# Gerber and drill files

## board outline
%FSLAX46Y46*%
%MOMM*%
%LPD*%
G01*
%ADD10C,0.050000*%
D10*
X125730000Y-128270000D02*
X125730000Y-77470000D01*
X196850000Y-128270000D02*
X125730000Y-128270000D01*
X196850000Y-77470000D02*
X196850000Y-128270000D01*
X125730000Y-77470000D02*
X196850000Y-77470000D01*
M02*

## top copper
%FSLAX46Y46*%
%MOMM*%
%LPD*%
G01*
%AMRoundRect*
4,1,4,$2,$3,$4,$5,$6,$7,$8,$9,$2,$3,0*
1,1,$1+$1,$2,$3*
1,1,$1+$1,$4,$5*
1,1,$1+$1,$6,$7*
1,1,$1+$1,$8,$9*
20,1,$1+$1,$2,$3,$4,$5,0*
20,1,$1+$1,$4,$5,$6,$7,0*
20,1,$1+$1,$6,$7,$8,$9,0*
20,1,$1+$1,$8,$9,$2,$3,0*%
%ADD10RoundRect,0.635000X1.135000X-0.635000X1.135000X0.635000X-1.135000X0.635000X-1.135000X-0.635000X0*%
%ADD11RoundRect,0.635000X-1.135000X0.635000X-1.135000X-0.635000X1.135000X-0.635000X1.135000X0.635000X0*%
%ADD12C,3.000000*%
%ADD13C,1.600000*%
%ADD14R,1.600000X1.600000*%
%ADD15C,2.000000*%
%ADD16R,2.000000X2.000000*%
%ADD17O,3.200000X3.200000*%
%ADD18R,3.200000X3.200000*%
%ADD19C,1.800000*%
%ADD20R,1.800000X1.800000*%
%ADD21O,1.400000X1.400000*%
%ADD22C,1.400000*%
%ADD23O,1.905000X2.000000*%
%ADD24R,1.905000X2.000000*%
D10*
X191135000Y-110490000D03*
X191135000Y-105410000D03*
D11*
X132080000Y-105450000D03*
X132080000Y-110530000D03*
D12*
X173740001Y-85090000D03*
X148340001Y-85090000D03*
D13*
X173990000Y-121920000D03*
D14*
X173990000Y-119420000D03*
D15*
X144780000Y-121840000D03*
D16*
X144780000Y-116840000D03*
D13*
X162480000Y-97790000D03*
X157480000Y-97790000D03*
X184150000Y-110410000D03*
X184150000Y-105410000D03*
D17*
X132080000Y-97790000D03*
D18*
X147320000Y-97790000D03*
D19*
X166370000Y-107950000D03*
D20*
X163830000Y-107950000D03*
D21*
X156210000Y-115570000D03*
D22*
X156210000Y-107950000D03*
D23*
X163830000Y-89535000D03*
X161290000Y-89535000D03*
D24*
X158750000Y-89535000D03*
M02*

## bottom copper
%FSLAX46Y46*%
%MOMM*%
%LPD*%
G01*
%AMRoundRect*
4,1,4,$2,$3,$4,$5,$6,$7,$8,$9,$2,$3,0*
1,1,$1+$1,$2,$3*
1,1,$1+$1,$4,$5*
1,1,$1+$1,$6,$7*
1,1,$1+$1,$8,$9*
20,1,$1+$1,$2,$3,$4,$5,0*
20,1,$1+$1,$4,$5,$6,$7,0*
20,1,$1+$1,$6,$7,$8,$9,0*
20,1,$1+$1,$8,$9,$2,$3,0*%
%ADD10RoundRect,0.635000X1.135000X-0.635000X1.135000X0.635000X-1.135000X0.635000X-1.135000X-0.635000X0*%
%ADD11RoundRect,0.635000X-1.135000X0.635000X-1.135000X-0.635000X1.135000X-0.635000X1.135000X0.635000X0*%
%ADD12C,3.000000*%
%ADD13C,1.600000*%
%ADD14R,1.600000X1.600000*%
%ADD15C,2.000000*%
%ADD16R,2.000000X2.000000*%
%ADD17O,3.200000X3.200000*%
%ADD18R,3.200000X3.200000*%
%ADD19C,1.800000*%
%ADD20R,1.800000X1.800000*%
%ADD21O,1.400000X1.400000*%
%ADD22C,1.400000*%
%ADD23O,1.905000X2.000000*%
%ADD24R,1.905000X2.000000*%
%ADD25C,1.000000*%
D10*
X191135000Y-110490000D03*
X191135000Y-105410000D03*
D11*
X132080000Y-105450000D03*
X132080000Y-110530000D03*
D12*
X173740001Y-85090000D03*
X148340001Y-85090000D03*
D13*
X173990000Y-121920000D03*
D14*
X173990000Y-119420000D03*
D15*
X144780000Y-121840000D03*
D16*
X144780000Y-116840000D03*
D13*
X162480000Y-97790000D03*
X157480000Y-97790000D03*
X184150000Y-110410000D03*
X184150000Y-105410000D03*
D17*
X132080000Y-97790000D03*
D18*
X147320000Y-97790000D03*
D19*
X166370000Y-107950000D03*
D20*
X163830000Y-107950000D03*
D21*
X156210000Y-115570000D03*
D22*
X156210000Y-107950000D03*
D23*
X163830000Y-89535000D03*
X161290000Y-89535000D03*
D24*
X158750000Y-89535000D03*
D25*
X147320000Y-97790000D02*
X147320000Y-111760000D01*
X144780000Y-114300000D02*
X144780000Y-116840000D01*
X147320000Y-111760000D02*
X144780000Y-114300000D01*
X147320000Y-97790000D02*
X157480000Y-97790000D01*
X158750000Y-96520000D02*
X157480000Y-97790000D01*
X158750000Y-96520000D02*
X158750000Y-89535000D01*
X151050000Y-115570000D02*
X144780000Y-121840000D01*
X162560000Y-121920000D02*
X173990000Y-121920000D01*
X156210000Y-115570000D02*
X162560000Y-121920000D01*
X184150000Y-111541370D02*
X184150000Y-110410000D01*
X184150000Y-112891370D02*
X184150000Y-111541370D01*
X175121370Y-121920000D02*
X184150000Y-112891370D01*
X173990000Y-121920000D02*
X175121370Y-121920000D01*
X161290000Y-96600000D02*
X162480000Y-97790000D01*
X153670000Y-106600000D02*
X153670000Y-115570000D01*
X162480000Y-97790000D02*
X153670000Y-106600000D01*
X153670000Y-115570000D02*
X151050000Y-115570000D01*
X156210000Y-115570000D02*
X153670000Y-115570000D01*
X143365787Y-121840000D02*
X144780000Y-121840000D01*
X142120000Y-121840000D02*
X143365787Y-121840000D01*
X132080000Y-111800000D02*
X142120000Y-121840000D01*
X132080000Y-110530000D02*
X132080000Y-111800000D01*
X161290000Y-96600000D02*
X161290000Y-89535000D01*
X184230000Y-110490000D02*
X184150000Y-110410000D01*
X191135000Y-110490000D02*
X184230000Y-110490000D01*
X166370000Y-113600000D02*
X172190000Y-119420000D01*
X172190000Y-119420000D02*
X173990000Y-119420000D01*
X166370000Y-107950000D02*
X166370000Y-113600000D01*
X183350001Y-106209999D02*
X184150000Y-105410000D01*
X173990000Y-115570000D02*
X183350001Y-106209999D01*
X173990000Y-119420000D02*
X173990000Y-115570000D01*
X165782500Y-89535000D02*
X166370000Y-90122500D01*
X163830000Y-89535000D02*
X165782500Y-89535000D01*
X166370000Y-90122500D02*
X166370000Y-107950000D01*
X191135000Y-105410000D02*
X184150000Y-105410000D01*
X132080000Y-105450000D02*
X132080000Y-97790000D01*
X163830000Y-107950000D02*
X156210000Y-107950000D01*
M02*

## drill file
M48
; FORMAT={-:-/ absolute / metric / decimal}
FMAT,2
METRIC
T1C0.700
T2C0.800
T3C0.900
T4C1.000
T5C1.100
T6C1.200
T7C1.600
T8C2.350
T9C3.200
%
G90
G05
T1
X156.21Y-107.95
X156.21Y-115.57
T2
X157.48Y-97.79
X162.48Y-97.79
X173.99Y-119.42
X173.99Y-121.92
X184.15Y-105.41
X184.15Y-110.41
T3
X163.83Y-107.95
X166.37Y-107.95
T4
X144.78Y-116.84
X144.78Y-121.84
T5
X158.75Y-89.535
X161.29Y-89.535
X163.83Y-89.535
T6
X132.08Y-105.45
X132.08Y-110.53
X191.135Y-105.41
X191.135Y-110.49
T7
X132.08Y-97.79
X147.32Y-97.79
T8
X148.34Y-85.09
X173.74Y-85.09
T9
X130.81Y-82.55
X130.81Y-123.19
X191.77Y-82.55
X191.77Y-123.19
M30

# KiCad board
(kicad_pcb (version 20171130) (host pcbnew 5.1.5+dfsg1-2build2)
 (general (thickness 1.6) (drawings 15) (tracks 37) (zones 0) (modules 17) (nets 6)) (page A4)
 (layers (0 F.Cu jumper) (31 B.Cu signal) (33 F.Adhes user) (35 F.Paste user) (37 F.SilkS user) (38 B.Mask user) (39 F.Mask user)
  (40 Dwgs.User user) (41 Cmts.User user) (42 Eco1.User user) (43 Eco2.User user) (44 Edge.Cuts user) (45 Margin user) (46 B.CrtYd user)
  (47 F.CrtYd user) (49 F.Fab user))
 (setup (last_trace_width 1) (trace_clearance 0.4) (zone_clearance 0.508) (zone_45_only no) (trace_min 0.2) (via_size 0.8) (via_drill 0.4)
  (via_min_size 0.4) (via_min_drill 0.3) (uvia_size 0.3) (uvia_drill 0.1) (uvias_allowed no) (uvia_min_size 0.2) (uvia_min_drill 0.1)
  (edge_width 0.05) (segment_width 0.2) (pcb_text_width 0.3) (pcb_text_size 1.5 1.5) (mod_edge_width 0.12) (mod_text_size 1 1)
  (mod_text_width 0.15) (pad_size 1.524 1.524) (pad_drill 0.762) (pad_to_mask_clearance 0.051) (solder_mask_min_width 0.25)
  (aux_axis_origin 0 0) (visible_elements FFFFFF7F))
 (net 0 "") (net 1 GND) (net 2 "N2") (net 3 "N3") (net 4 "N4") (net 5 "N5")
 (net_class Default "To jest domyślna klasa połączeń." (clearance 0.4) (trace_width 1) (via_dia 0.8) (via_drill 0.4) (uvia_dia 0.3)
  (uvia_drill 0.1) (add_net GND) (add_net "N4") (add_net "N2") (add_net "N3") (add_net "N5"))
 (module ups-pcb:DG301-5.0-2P (layer F.Cu) (at 191.135 107.99 90)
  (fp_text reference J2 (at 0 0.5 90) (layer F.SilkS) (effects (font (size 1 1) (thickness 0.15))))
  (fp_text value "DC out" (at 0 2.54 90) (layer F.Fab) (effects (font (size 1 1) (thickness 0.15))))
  (pad 1 thru_hole roundrect (at -2.5 0 90) (size 2.54 3.54) (drill 1.2) (layers *.Cu *.Mask) (roundrect_rratio 0.25) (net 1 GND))
  (pad 2 thru_hole roundrect (at 2.58 0 90) (size 2.54 3.54) (drill 1.2) (layers *.Cu *.Mask) (roundrect_rratio 0.25) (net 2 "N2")))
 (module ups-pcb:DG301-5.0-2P (layer F.Cu) (at 132.08 107.95 270)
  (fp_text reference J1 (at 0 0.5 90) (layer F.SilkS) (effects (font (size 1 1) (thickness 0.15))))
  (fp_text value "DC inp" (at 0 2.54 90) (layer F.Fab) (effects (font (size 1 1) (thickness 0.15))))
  (pad 1 thru_hole roundrect (at -2.5 0 270) (size 2.54 3.54) (drill 1.2) (layers *.Cu *.Mask) (roundrect_rratio 0.25) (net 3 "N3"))
  (pad 2 thru_hole roundrect (at 2.58 0 270) (size 2.54 3.54) (drill 1.2) (layers *.Cu *.Mask) (roundrect_rratio 0.25) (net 1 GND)))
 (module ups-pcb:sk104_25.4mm (layer F.Cu) (at 161.040001 85.09)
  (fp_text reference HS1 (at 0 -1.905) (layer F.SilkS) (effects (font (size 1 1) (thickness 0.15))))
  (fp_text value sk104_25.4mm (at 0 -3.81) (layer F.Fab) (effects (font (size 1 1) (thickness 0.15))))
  (pad "" np_thru_hole circle (at 12.7 0) (size 3 3) (drill 2.35) (layers *.Cu *.Mask))
  (pad "" np_thru_hole circle (at -12.7 0) (size 3 3) (drill 2.35) (layers *.Cu *.Mask)))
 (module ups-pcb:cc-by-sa (layer F.Cu) (at 159.385 121.92)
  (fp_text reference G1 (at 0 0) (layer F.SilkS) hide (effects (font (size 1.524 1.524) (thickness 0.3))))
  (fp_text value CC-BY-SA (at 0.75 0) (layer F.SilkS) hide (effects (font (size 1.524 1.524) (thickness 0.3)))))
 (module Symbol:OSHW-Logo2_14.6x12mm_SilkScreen (layer F.Cu) (at 186.055 93.98)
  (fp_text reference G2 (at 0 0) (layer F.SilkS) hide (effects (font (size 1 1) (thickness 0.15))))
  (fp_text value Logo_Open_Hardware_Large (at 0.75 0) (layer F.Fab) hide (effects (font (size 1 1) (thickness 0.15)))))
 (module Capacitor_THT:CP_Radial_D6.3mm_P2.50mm (layer F.Cu) (at 173.99 119.42 270)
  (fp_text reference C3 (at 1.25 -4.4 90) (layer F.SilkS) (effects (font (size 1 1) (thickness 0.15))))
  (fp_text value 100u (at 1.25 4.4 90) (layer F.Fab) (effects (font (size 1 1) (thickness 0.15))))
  (pad 2 thru_hole circle (at 2.5 0 270) (size 1.6 1.6) (drill 0.8) (layers *.Cu *.Mask) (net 1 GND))
  (pad 1 thru_hole rect (at 0 0 270) (size 1.6 1.6) (drill 0.8) (layers *.Cu *.Mask) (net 2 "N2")))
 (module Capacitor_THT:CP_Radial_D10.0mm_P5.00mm (layer F.Cu) (at 144.78 116.84 270)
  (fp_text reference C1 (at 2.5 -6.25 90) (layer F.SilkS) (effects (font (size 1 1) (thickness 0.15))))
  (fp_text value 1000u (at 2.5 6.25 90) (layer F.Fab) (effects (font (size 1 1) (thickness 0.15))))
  (pad 2 thru_hole circle (at 5 0 270) (size 2 2) (drill 1) (layers *.Cu *.Mask) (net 1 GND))
  (pad 1 thru_hole rect (at 0 0 270) (size 2 2) (drill 1) (layers *.Cu *.Mask) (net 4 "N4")))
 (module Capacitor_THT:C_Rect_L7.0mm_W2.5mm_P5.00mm (layer F.Cu) (at 157.48 97.79)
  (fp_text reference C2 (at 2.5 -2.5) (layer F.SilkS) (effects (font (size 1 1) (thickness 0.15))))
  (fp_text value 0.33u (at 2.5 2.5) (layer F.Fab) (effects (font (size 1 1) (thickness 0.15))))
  (pad 2 thru_hole circle (at 5 0) (size 1.6 1.6) (drill 0.8) (layers *.Cu *.Mask) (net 1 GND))
  (pad 1 thru_hole circle (at 0 0) (size 1.6 1.6) (drill 0.8) (layers *.Cu *.Mask) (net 4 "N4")))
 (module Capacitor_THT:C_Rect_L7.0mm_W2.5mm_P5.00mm (layer F.Cu) (at 184.15 105.41 270)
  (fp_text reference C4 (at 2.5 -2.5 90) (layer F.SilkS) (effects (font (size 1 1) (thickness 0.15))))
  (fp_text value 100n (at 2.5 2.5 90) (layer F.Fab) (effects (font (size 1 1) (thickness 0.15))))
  (pad 2 thru_hole circle (at 5 0 270) (size 1.6 1.6) (drill 0.8) (layers *.Cu *.Mask) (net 1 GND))
  (pad 1 thru_hole circle (at 0 0 270) (size 1.6 1.6) (drill 0.8) (layers *.Cu *.Mask) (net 2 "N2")))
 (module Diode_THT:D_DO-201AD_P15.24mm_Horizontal (layer F.Cu) (at 147.32 97.79 180)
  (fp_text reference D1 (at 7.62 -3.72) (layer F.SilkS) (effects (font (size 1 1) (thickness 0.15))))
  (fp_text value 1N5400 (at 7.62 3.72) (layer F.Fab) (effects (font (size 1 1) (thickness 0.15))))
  (pad 2 thru_hole oval (at 15.24 0 180) (size 3.2 3.2) (drill 1.6) (layers *.Cu *.Mask) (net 3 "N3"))
  (pad 1 thru_hole rect (at 0 0 180) (size 3.2 3.2) (drill 1.6) (layers *.Cu *.Mask) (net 4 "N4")))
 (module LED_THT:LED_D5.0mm (layer F.Cu) (at 163.83 107.95)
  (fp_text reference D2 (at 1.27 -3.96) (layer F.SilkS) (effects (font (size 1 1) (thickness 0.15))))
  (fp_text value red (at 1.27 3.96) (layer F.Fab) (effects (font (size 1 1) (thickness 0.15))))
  (pad 2 thru_hole circle (at 2.54 0) (size 1.8 1.8) (drill 0.9) (layers *.Cu *.Mask) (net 2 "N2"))
  (pad 1 thru_hole rect (at 0 0) (size 1.8 1.8) (drill 0.9) (layers *.Cu *.Mask) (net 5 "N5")))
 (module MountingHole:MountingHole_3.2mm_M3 (layer F.Cu) (at 130.81 82.55)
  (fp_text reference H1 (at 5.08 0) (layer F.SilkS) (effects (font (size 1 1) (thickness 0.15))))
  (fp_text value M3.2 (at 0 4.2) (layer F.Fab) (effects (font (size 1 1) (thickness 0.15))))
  (pad 1 np_thru_hole circle (at 0 0) (size 3.2 3.2) (drill 3.2) (layers *.Cu *.Mask)))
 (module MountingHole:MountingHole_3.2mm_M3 (layer F.Cu) (at 191.77 82.55)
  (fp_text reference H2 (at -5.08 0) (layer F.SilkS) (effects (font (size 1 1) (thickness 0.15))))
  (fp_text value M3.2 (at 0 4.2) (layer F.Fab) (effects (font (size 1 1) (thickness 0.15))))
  (pad 1 np_thru_hole circle (at 0 0) (size 3.2 3.2) (drill 3.2) (layers *.Cu *.Mask)))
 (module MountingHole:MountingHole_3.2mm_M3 (layer F.Cu) (at 191.77 123.19)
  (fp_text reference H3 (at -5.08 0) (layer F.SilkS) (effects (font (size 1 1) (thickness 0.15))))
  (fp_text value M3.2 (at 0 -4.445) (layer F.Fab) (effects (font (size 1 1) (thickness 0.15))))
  (pad 1 np_thru_hole circle (at 0 0) (size 3.2 3.2) (drill 3.2) (layers *.Cu *.Mask)))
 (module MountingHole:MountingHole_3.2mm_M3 (layer F.Cu) (at 130.81 123.19)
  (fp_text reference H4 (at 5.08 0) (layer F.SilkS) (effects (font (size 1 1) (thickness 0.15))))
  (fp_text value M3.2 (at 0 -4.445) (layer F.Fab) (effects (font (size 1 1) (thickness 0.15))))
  (pad 1 np_thru_hole circle (at 0 0) (size 3.2 3.2) (drill 3.2) (layers *.Cu *.Mask)))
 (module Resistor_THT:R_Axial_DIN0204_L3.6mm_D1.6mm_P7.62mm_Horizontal (layer F.Cu) (at 156.21 107.95 270)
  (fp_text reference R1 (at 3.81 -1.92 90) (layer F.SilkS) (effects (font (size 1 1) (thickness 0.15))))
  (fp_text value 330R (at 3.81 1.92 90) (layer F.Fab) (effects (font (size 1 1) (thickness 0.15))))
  (pad 2 thru_hole oval (at 7.62 0 270) (size 1.4 1.4) (drill 0.7) (layers *.Cu *.Mask) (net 1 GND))
  (pad 1 thru_hole circle (at 0 0 270) (size 1.4 1.4) (drill 0.7) (layers *.Cu *.Mask) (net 5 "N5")))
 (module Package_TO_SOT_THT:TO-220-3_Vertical (layer F.Cu) (at 158.75 89.535)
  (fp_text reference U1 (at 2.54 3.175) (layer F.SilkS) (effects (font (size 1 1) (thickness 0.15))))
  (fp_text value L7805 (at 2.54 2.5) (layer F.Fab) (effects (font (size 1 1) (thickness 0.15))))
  (pad 3 thru_hole oval (at 5.08 0) (size 1.905 2) (drill 1.1) (layers *.Cu *.Mask) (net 2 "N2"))
  (pad 2 thru_hole oval (at 2.54 0) (size 1.905 2) (drill 1.1) (layers *.Cu *.Mask) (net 1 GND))
  (pad 1 thru_hole rect (at 0 0) (size 1.905 2) (drill 1.1) (layers *.Cu *.Mask) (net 4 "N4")))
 (gr_line (start 125.73 128.27) (end 125.73 77.47) (layer Edge.Cuts) (width 0.05))
 (gr_line (start 196.85 128.27) (end 125.73 128.27) (layer Edge.Cuts) (width 0.05))
 (gr_line (start 196.85 77.47) (end 196.85 128.27) (layer Edge.Cuts) (width 0.05))
 (gr_line (start 125.73 77.47) (end 196.85 77.47) (layer Edge.Cuts) (width 0.05))
 (segment (start 147.32 97.79) (end 147.32 111.76) (width 1) (layer B.Cu) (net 4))
 (segment (start 144.78 114.3) (end 144.78 116.84) (width 1) (layer B.Cu) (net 4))
 (segment (start 147.32 111.76) (end 144.78 114.3) (width 1) (layer B.Cu) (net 4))
 (segment (start 147.32 97.79) (end 157.48 97.79) (width 1) (layer B.Cu) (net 4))
 (segment (start 158.75 96.52) (end 157.48 97.79) (width 1) (layer B.Cu) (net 4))
 (segment (start 158.75 96.52) (end 158.75 89.535) (width 1) (layer B.Cu) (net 4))
 (segment (start 151.05 115.57) (end 144.78 121.84) (width 1) (layer B.Cu) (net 1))
 (segment (start 162.56 121.92) (end 173.99 121.92) (width 1) (layer B.Cu) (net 1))
 (segment (start 156.21 115.57) (end 162.56 121.92) (width 1) (layer B.Cu) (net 1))
 (segment (start 184.15 111.54137) (end 184.15 110.41) (width 1) (layer B.Cu) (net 1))
 (segment (start 184.15 112.89137) (end 184.15 111.54137) (width 1) (layer B.Cu) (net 1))
 (segment (start 175.12137 121.92) (end 184.15 112.89137) (width 1) (layer B.Cu) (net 1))
 (segment (start 173.99 121.92) (end 175.12137 121.92) (width 1) (layer B.Cu) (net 1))
 (segment (start 161.29 96.6) (end 162.48 97.79) (width 1) (layer B.Cu) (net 1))
 (segment (start 153.67 106.6) (end 153.67 115.57) (width 1) (layer B.Cu) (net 1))
 (segment (start 162.48 97.79) (end 153.67 106.6) (width 1) (layer B.Cu) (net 1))
 (segment (start 153.67 115.57) (end 151.05 115.57) (width 1) (layer B.Cu) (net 1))
 (segment (start 156.21 115.57) (end 153.67 115.57) (width 1) (layer B.Cu) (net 1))
 (segment (start 143.365787 121.84) (end 144.78 121.84) (width 1) (layer B.Cu) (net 1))
 (segment (start 142.12 121.84) (end 143.365787 121.84) (width 1) (layer B.Cu) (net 1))
 (segment (start 132.08 111.8) (end 142.12 121.84) (width 1) (layer B.Cu) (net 1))
 (segment (start 132.08 110.53) (end 132.08 111.8) (width 1) (layer B.Cu) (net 1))
 (segment (start 161.29 96.6) (end 161.29 89.535) (width 1) (layer B.Cu) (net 1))
 (segment (start 184.23 110.49) (end 184.15 110.41) (width 1) (layer B.Cu) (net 1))
 (segment (start 191.135 110.49) (end 184.23 110.49) (width 1) (layer B.Cu) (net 1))
 (segment (start 166.37 113.6) (end 172.19 119.42) (width 1) (layer B.Cu) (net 2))
 (segment (start 172.19 119.42) (end 173.99 119.42) (width 1) (layer B.Cu) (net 2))
 (segment (start 166.37 107.95) (end 166.37 113.6) (width 1) (layer B.Cu) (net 2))
 (segment (start 183.350001 106.209999) (end 184.15 105.41) (width 1) (layer B.Cu) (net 2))
 (segment (start 173.99 115.57) (end 183.350001 106.209999) (width 1) (layer B.Cu) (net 2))
 (segment (start 173.99 119.42) (end 173.99 115.57) (width 1) (layer B.Cu) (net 2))
 (segment (start 165.7825 89.535) (end 166.37 90.1225) (width 1) (layer B.Cu) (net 2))
 (segment (start 163.83 89.535) (end 165.7825 89.535) (width 1) (layer B.Cu) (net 2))
 (segment (start 166.37 90.1225) (end 166.37 107.95) (width 1) (layer B.Cu) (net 2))
 (segment (start 191.135 105.41) (end 184.15 105.41) (width 1) (layer B.Cu) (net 2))
 (segment (start 132.08 105.45) (end 132.08 97.79) (width 1) (layer B.Cu) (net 3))
 (segment (start 163.83 107.95) (end 156.21 107.95) (width 1) (layer B.Cu) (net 5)))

